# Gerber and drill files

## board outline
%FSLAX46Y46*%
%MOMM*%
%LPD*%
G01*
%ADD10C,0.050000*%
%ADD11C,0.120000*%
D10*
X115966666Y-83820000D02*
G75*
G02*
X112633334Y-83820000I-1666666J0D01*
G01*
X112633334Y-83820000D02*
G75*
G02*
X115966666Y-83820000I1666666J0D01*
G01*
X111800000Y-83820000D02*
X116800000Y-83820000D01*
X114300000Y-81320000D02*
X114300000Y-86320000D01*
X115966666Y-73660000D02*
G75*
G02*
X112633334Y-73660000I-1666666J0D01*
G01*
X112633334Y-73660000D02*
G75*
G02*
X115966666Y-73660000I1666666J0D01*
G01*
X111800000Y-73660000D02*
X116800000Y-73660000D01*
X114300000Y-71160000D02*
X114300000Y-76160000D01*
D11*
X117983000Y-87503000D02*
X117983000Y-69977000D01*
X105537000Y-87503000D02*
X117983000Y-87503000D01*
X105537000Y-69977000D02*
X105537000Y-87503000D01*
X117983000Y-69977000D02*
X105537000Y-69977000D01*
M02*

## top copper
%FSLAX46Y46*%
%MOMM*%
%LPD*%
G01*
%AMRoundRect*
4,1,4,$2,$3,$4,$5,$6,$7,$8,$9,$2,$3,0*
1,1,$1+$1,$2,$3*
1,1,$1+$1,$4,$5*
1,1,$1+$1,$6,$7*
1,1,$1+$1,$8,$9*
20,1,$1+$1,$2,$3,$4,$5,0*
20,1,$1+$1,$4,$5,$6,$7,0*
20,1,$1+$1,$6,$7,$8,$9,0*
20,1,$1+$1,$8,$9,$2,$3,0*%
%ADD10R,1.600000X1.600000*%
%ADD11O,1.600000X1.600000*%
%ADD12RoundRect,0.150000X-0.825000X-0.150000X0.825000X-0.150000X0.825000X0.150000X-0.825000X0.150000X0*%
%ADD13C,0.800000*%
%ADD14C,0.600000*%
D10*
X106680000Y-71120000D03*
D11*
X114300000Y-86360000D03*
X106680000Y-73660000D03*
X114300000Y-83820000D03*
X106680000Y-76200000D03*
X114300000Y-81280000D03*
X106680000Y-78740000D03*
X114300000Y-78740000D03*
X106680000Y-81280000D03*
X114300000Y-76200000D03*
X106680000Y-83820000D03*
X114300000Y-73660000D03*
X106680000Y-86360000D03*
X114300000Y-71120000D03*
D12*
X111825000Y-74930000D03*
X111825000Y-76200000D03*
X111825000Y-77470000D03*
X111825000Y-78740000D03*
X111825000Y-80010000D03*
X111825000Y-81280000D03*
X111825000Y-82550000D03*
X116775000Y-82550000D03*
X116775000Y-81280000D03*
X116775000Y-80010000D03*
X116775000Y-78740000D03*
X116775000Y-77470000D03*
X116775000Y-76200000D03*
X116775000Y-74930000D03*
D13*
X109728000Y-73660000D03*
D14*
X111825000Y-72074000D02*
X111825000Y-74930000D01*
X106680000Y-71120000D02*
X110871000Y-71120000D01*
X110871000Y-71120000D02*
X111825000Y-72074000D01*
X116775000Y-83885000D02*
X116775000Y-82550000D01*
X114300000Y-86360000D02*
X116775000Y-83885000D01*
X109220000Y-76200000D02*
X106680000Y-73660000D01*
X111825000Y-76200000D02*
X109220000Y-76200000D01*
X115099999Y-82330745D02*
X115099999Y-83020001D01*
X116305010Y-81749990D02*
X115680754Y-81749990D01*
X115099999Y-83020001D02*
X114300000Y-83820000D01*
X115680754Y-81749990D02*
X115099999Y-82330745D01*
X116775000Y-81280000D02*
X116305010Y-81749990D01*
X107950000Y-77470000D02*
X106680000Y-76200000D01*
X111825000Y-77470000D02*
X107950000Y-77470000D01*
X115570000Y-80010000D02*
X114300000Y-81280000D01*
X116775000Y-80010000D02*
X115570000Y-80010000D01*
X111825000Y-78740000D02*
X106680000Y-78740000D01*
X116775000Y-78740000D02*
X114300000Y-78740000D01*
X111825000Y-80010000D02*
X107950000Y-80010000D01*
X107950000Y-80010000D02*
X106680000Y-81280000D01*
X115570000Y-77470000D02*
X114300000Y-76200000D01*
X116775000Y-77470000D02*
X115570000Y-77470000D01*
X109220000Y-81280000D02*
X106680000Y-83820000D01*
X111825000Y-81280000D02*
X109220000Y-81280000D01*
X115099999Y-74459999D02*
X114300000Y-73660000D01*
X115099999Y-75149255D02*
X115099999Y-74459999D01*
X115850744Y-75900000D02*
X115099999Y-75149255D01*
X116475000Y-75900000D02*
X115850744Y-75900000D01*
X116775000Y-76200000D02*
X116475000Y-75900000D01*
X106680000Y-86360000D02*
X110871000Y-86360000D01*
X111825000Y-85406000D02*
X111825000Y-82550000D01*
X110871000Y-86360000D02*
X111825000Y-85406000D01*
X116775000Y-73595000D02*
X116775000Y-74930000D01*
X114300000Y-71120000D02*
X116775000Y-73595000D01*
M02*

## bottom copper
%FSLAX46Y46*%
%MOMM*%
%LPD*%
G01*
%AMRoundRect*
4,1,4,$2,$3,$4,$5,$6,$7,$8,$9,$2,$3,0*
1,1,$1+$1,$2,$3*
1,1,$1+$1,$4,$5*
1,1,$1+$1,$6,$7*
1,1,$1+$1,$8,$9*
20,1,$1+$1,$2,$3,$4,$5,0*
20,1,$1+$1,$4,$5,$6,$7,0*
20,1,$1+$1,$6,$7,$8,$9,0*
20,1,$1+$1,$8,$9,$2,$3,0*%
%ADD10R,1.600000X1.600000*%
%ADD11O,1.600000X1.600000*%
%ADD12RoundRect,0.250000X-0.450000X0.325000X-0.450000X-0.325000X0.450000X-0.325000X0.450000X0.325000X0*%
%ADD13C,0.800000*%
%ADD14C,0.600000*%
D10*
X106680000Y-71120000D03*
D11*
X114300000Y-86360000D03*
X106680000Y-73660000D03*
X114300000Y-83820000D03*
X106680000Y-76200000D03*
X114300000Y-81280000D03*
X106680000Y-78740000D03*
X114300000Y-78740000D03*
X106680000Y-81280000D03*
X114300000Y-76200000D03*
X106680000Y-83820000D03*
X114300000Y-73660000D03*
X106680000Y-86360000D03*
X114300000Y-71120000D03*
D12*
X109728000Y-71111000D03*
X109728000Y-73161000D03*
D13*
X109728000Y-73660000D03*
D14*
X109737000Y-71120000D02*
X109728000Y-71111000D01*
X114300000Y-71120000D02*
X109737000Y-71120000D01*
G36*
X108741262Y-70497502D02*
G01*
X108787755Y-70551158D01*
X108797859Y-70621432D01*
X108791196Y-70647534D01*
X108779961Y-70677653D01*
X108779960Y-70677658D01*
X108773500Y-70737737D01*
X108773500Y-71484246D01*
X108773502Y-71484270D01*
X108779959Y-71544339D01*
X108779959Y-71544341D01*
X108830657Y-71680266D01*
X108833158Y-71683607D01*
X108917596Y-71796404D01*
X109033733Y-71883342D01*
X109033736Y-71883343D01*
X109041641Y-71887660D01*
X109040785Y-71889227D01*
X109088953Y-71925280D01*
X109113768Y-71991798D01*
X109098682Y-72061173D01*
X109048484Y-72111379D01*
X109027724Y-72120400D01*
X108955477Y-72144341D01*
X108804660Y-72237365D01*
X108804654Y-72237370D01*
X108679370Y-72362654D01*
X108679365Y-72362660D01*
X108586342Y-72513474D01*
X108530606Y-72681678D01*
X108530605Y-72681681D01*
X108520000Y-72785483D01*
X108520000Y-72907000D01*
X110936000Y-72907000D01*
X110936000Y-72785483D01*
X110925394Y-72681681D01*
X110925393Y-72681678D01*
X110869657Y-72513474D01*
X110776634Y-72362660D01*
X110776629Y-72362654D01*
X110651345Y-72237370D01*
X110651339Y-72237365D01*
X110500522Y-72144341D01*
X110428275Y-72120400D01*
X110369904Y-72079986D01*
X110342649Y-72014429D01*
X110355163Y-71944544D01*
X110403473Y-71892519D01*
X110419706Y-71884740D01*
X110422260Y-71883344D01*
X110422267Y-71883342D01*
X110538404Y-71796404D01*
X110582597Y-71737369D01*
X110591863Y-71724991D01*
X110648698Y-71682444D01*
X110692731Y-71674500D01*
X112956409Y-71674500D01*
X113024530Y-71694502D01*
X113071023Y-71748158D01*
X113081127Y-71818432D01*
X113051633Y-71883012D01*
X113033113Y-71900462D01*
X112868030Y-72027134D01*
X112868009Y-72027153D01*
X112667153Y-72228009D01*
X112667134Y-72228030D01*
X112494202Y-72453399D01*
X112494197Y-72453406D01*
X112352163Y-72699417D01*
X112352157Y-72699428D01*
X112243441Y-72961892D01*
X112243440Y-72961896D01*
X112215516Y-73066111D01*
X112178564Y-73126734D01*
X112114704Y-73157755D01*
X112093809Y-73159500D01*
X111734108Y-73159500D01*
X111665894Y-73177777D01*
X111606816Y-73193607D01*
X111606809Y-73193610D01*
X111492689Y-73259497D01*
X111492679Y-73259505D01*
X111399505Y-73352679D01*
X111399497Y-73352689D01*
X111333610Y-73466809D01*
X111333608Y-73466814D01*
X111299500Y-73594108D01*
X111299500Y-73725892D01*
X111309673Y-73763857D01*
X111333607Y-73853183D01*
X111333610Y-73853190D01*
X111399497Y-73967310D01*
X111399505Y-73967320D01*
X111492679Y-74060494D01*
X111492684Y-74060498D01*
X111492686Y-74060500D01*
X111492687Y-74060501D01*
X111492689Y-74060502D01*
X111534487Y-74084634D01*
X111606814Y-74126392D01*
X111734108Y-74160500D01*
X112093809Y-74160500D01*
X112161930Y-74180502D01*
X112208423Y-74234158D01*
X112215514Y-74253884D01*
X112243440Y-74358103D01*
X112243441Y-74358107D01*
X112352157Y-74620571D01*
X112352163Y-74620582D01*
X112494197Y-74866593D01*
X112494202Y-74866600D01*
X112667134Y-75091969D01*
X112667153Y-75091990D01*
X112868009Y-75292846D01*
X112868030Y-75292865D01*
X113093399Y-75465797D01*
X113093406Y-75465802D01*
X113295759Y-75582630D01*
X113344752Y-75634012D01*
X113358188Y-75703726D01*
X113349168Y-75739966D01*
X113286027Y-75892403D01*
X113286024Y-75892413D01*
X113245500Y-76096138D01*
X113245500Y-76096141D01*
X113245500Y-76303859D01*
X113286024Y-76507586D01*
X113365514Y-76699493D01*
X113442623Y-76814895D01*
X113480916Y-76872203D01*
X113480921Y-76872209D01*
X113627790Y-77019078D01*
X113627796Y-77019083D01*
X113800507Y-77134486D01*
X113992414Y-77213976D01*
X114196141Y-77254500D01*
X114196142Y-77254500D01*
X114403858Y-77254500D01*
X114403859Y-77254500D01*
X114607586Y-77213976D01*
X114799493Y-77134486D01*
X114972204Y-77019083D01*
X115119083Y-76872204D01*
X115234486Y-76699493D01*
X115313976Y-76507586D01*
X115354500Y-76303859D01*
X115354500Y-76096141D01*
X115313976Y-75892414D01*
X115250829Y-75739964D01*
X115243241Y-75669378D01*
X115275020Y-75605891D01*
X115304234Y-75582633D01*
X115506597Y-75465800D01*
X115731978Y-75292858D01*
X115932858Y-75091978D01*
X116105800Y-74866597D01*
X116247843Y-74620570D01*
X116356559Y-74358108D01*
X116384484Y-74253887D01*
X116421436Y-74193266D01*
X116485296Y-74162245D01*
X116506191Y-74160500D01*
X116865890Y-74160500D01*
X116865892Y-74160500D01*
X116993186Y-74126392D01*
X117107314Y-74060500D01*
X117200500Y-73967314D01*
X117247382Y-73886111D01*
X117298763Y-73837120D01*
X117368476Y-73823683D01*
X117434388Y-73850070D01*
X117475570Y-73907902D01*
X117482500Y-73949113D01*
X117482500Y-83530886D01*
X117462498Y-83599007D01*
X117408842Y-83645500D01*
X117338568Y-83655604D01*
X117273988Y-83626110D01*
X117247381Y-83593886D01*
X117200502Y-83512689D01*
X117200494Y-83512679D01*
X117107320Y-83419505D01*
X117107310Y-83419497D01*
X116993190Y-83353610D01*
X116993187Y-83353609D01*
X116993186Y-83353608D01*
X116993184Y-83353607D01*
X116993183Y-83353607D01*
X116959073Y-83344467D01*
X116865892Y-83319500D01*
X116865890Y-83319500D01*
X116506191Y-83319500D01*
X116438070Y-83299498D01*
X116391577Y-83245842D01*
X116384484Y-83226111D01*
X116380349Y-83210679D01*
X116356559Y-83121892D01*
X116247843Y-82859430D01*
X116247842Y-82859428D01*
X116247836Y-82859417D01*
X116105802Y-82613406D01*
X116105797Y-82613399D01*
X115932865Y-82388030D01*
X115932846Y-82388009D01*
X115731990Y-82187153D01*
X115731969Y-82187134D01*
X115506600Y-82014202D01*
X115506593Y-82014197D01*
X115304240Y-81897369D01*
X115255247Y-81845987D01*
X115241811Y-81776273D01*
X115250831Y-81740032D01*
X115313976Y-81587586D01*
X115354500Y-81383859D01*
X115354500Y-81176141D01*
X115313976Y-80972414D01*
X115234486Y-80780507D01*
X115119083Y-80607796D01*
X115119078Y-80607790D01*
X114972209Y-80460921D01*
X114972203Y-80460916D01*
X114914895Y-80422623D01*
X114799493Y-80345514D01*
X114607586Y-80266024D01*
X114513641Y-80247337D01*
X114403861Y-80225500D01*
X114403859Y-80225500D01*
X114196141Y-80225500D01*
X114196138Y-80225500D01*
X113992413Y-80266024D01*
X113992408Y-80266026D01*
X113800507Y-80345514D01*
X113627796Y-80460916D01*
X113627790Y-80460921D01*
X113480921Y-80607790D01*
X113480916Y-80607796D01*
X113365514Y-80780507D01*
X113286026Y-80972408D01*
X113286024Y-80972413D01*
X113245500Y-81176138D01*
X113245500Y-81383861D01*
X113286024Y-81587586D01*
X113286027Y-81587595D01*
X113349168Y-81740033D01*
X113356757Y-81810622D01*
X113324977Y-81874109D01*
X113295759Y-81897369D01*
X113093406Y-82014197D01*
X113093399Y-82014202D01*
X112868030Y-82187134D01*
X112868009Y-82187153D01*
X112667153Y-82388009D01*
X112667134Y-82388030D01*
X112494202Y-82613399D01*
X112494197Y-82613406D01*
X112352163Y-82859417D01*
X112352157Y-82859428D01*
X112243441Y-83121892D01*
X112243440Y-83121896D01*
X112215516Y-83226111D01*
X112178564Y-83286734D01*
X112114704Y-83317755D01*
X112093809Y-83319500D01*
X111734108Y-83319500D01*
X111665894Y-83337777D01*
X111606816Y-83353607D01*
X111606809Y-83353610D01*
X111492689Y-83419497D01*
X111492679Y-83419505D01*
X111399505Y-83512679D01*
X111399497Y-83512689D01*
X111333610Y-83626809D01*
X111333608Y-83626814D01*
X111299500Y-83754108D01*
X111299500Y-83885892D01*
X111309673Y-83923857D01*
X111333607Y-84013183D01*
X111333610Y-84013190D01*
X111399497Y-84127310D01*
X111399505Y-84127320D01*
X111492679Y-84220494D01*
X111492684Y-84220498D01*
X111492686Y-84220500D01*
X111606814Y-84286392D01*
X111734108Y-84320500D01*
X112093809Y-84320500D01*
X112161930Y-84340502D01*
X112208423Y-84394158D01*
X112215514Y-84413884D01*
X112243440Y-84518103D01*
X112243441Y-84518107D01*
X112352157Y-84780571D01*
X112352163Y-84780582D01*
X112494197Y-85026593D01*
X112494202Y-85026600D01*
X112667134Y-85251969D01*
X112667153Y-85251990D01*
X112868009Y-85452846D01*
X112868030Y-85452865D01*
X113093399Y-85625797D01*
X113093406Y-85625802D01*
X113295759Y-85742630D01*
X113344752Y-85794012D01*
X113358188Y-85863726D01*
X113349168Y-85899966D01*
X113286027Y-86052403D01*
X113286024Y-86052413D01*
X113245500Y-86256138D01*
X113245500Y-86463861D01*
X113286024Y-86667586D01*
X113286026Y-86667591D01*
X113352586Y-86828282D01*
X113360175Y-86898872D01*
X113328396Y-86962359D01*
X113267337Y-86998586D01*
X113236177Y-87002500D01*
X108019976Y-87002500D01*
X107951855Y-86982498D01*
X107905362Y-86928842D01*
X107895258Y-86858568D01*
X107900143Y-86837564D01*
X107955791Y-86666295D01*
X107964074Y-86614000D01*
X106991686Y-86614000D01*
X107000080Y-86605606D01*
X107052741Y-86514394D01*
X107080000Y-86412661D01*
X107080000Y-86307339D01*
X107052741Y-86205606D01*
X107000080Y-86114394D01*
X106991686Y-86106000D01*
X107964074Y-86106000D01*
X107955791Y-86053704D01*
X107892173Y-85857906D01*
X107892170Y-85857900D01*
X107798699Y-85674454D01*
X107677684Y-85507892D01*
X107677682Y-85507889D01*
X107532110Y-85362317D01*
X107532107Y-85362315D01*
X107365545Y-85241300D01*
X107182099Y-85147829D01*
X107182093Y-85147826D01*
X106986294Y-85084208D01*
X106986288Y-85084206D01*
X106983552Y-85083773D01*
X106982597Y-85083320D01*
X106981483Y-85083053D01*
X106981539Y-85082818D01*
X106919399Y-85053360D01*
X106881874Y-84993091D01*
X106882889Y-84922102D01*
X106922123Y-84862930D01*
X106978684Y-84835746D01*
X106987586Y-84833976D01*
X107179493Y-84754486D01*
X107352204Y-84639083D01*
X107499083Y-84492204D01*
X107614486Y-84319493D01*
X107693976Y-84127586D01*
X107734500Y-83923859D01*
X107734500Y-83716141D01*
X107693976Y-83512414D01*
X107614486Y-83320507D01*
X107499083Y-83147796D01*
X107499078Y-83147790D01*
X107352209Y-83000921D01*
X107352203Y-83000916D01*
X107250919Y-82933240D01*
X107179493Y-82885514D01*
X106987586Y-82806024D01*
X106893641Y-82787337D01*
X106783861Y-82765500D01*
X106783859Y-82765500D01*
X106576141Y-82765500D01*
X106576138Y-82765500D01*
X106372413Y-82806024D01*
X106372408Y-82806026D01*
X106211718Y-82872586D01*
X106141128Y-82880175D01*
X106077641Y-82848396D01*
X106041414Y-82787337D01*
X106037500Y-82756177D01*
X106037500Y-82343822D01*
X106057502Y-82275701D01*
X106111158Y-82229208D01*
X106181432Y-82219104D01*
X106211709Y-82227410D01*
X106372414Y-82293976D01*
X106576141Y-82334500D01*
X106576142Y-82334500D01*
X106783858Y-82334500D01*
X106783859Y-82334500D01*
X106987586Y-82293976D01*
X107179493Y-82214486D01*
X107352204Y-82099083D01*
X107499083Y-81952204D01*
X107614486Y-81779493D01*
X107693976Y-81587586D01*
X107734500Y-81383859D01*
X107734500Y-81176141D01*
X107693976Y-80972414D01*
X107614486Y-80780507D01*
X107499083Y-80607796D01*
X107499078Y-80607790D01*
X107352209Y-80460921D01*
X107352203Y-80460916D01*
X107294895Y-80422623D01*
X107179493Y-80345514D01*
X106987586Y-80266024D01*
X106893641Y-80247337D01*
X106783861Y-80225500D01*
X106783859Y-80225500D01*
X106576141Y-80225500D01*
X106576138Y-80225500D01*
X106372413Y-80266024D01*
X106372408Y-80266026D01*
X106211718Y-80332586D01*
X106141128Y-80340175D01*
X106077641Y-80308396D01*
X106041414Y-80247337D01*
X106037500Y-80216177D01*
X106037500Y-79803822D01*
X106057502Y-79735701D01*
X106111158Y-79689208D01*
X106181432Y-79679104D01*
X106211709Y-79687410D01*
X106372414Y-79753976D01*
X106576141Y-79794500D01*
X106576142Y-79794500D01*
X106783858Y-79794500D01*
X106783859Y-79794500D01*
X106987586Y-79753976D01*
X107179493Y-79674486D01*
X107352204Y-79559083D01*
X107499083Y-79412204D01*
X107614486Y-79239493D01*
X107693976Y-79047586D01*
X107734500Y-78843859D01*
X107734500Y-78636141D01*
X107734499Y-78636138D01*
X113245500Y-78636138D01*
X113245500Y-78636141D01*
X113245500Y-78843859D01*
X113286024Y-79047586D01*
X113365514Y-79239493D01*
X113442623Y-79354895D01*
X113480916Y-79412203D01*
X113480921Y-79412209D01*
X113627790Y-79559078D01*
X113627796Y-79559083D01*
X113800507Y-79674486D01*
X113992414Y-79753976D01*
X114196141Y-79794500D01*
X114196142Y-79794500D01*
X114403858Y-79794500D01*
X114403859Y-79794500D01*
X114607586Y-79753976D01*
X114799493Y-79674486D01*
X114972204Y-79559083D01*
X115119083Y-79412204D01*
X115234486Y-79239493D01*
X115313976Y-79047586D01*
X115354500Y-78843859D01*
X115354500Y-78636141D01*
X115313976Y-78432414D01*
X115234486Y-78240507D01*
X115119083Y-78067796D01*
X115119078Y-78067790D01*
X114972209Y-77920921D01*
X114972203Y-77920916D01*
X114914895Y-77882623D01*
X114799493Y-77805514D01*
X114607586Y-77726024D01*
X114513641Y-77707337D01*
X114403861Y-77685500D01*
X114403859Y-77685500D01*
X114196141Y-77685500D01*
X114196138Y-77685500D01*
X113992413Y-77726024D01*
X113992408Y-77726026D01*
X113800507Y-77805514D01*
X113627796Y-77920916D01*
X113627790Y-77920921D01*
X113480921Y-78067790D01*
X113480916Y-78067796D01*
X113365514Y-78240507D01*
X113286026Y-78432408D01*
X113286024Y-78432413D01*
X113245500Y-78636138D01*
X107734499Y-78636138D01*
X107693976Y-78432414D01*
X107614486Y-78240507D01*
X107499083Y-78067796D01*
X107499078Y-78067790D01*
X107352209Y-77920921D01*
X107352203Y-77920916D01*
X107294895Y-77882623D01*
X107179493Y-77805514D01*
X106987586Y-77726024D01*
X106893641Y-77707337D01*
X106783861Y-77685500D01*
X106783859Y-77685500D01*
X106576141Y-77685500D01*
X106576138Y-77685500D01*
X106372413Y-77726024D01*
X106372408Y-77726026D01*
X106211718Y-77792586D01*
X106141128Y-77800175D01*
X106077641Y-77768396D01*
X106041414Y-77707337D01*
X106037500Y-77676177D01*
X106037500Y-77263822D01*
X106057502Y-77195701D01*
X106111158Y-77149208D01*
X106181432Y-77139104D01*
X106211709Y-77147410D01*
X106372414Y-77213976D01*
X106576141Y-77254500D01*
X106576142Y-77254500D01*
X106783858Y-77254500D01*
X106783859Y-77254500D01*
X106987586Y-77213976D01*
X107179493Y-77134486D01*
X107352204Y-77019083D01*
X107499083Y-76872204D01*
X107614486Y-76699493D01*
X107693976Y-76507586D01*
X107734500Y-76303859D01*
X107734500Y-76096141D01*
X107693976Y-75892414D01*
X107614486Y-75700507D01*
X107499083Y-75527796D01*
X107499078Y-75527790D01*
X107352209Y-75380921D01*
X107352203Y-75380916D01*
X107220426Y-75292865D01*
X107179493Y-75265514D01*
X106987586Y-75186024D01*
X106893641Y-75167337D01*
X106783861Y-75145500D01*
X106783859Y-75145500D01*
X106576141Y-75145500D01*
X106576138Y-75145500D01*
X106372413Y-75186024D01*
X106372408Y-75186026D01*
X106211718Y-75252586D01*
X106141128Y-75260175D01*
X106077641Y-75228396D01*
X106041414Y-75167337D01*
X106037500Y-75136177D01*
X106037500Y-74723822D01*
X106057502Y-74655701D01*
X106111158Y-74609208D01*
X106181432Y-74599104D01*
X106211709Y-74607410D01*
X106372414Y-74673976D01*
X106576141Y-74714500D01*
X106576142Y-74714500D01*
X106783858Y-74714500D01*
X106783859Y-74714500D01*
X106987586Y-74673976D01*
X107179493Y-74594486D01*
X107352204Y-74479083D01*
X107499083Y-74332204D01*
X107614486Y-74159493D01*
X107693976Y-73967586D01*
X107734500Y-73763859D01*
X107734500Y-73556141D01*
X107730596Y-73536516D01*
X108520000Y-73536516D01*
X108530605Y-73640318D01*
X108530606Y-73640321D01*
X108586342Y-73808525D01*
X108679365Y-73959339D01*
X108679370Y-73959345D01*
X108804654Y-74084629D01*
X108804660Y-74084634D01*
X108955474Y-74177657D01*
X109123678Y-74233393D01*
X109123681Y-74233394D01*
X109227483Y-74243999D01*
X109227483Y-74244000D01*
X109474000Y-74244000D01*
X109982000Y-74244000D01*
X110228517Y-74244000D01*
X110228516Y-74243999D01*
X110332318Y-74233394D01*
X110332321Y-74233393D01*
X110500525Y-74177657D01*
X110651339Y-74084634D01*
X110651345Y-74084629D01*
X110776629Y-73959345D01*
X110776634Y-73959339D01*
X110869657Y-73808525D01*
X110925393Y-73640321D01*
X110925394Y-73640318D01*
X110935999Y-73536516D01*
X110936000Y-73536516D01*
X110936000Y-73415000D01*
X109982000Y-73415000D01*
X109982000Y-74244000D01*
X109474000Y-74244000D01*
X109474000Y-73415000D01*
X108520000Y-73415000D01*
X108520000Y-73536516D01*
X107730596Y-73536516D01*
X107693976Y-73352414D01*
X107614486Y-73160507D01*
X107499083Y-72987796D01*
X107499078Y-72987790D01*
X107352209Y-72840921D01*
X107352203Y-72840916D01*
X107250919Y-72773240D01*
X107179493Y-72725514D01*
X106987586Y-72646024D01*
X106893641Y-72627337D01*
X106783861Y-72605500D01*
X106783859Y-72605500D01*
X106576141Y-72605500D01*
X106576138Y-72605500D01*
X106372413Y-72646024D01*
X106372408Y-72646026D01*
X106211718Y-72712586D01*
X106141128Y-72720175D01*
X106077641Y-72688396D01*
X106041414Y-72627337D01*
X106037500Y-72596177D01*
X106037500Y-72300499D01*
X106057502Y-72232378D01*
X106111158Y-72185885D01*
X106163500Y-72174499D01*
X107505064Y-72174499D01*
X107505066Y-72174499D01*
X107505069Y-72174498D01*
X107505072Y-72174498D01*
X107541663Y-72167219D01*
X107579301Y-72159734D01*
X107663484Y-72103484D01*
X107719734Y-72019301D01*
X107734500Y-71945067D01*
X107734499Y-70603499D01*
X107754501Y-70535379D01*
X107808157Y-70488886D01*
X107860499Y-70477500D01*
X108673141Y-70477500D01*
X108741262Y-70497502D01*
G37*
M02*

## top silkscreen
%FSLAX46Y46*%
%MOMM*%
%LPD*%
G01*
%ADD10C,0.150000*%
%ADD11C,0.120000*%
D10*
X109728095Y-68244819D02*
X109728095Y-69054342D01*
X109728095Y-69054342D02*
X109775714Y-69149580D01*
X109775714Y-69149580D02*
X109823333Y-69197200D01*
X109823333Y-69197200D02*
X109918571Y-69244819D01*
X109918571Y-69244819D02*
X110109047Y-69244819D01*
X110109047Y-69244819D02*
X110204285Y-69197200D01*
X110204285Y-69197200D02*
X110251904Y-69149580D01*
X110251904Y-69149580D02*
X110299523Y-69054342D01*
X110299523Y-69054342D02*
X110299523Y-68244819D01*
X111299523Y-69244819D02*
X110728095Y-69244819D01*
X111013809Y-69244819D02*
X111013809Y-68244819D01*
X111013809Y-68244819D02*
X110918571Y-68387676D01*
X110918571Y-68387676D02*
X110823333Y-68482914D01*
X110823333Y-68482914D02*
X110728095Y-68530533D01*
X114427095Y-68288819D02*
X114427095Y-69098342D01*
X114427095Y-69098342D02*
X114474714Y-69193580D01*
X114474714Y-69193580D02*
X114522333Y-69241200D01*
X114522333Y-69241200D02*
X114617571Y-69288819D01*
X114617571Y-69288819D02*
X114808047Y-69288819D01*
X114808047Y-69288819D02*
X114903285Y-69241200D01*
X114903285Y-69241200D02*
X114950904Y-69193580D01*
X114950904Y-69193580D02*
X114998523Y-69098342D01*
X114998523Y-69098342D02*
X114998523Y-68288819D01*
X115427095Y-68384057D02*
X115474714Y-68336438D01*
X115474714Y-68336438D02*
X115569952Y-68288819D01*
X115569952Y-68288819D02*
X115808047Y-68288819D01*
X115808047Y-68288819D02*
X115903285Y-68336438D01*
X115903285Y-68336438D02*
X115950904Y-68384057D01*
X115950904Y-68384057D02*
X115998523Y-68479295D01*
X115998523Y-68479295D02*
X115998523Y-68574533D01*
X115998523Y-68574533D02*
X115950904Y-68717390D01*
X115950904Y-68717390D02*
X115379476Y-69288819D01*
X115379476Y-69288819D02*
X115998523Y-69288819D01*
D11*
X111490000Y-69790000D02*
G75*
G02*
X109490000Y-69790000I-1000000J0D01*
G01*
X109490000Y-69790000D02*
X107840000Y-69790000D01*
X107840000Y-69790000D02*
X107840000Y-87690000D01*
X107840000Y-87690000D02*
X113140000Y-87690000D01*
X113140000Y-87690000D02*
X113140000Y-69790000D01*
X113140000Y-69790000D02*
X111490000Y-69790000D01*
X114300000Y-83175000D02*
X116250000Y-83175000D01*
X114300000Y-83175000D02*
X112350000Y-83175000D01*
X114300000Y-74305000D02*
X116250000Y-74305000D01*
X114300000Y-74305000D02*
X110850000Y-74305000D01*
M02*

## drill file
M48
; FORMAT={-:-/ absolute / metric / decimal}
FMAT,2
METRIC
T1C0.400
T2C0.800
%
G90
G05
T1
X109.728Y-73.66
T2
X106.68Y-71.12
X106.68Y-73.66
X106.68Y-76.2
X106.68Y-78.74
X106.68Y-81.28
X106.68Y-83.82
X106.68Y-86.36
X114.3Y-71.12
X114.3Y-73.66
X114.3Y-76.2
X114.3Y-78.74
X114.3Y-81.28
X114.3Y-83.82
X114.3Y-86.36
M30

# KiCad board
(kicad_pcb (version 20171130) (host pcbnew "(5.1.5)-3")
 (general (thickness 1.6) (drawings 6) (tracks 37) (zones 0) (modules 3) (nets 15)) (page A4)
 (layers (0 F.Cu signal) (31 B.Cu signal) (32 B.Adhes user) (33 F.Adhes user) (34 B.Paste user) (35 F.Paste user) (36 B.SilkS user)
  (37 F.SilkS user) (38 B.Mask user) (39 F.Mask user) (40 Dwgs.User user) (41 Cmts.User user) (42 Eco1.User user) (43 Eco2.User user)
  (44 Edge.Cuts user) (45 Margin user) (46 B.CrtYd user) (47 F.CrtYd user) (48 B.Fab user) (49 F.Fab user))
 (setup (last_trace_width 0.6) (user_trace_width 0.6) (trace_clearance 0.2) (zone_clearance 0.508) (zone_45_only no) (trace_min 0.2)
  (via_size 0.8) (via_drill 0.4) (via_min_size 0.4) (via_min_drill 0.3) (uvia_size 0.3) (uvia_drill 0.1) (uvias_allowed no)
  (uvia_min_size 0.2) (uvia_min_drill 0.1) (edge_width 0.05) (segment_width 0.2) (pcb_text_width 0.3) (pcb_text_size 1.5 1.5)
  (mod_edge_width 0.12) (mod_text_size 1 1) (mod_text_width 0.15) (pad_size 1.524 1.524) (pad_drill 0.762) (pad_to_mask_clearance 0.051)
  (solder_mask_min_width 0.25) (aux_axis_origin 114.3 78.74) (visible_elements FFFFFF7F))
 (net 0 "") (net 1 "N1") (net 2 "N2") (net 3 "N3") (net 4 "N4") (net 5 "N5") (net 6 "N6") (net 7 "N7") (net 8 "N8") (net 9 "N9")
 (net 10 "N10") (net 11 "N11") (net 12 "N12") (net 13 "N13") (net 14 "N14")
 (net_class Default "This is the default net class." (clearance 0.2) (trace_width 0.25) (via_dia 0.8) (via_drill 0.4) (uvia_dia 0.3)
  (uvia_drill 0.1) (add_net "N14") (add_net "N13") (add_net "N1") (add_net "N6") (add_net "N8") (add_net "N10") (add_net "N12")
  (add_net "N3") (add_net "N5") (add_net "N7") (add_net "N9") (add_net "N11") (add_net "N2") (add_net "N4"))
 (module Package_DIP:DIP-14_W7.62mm (layer F.Cu) (at 106.68 71.12)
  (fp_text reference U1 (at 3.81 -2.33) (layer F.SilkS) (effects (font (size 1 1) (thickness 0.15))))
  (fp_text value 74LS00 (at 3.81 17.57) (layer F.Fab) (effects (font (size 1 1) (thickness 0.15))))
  (fp_arc (start 3.81 -1.33) (end 2.81 -1.33) (angle -180) (layer F.SilkS) (width 0.12))
  (fp_line (start 2.81 -1.33) (end 1.16 -1.33) (layer F.SilkS) (width 0.12))
  (fp_line (start 1.16 -1.33) (end 1.16 16.57) (layer F.SilkS) (width 0.12))
  (fp_line (start 1.16 16.57) (end 6.46 16.57) (layer F.SilkS) (width 0.12))
  (fp_line (start 6.46 16.57) (end 6.46 -1.33) (layer F.SilkS) (width 0.12))
  (fp_line (start 6.46 -1.33) (end 4.81 -1.33) (layer F.SilkS) (width 0.12))
  (pad 1 thru_hole rect (at 0 0) (size 1.6 1.6) (drill 0.8) (layers *.Cu *.Mask) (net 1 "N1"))
  (pad 8 thru_hole oval (at 7.62 15.24) (size 1.6 1.6) (drill 0.8) (layers *.Cu *.Mask) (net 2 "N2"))
  (pad 2 thru_hole oval (at 0 2.54) (size 1.6 1.6) (drill 0.8) (layers *.Cu *.Mask) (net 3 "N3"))
  (pad 9 thru_hole oval (at 7.62 12.7) (size 1.6 1.6) (drill 0.8) (layers *.Cu *.Mask) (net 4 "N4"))
  (pad 3 thru_hole oval (at 0 5.08) (size 1.6 1.6) (drill 0.8) (layers *.Cu *.Mask) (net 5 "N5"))
  (pad 10 thru_hole oval (at 7.62 10.16) (size 1.6 1.6) (drill 0.8) (layers *.Cu *.Mask) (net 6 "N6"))
  (pad 4 thru_hole oval (at 0 7.62) (size 1.6 1.6) (drill 0.8) (layers *.Cu *.Mask) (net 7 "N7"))
  (pad 11 thru_hole oval (at 7.62 7.62) (size 1.6 1.6) (drill 0.8) (layers *.Cu *.Mask) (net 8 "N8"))
  (pad 5 thru_hole oval (at 0 10.16) (size 1.6 1.6) (drill 0.8) (layers *.Cu *.Mask) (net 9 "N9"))
  (pad 12 thru_hole oval (at 7.62 5.08) (size 1.6 1.6) (drill 0.8) (layers *.Cu *.Mask) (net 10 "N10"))
  (pad 6 thru_hole oval (at 0 12.7) (size 1.6 1.6) (drill 0.8) (layers *.Cu *.Mask) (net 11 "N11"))
  (pad 13 thru_hole oval (at 7.62 2.54) (size 1.6 1.6) (drill 0.8) (layers *.Cu *.Mask) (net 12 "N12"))
  (pad 7 thru_hole oval (at 0 15.24) (size 1.6 1.6) (drill 0.8) (layers *.Cu *.Mask) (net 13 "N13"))
  (pad 14 thru_hole oval (at 7.62 0) (size 1.6 1.6) (drill 0.8) (layers *.Cu *.Mask) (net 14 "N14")))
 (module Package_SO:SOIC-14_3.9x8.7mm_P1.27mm (layer F.Cu) (at 114.3 78.74)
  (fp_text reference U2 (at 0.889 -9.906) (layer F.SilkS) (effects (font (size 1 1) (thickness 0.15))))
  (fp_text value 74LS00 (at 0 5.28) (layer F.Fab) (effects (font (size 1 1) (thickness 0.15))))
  (fp_line (start 0 4.435) (end 1.95 4.435) (layer F.SilkS) (width 0.12))
  (fp_line (start 0 4.435) (end -1.95 4.435) (layer F.SilkS) (width 0.12))
  (fp_line (start 0 -4.435) (end 1.95 -4.435) (layer F.SilkS) (width 0.12))
  (fp_line (start 0 -4.435) (end -3.45 -4.435) (layer F.SilkS) (width 0.12))
  (pad 1 smd roundrect (at -2.475 -3.81) (size 1.95 0.6) (layers F.Cu F.Paste F.Mask) (roundrect_rratio 0.25) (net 1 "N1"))
  (pad 2 smd roundrect (at -2.475 -2.54) (size 1.95 0.6) (layers F.Cu F.Paste F.Mask) (roundrect_rratio 0.25) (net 3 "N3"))
  (pad 3 smd roundrect (at -2.475 -1.27) (size 1.95 0.6) (layers F.Cu F.Paste F.Mask) (roundrect_rratio 0.25) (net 5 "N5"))
  (pad 4 smd roundrect (at -2.475 0) (size 1.95 0.6) (layers F.Cu F.Paste F.Mask) (roundrect_rratio 0.25) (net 7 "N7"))
  (pad 5 smd roundrect (at -2.475 1.27) (size 1.95 0.6) (layers F.Cu F.Paste F.Mask) (roundrect_rratio 0.25) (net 9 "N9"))
  (pad 6 smd roundrect (at -2.475 2.54) (size 1.95 0.6) (layers F.Cu F.Paste F.Mask) (roundrect_rratio 0.25) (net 11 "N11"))
  (pad 7 smd roundrect (at -2.475 3.81) (size 1.95 0.6) (layers F.Cu F.Paste F.Mask) (roundrect_rratio 0.25) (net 13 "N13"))
  (pad 8 smd roundrect (at 2.475 3.81) (size 1.95 0.6) (layers F.Cu F.Paste F.Mask) (roundrect_rratio 0.25) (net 2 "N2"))
  (pad 9 smd roundrect (at 2.475 2.54) (size 1.95 0.6) (layers F.Cu F.Paste F.Mask) (roundrect_rratio 0.25) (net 4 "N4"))
  (pad 10 smd roundrect (at 2.475 1.27) (size 1.95 0.6) (layers F.Cu F.Paste F.Mask) (roundrect_rratio 0.25) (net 6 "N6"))
  (pad 11 smd roundrect (at 2.475 0) (size 1.95 0.6) (layers F.Cu F.Paste F.Mask) (roundrect_rratio 0.25) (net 8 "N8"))
  (pad 12 smd roundrect (at 2.475 -1.27) (size 1.95 0.6) (layers F.Cu F.Paste F.Mask) (roundrect_rratio 0.25) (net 10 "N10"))
  (pad 13 smd roundrect (at 2.475 -2.54) (size 1.95 0.6) (layers F.Cu F.Paste F.Mask) (roundrect_rratio 0.25) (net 12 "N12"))
  (pad 14 smd roundrect (at 2.475 -3.81) (size 1.95 0.6) (layers F.Cu F.Paste F.Mask) (roundrect_rratio 0.25) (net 14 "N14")))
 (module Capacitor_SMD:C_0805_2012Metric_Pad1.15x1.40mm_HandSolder (layer B.Cu) (at 109.728 72.136 270)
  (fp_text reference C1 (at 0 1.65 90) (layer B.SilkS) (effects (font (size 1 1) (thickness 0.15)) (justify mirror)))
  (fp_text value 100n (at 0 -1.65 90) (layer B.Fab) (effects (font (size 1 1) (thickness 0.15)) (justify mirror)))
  (pad 1 smd roundrect (at -1.025 0 270) (size 1.15 1.4) (layers B.Cu B.Paste B.Mask) (roundrect_rratio 0.217391) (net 14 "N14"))
  (pad 2 smd roundrect (at 1.025 0 270) (size 1.15 1.4) (layers B.Cu B.Paste B.Mask) (roundrect_rratio 0.217391) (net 13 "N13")))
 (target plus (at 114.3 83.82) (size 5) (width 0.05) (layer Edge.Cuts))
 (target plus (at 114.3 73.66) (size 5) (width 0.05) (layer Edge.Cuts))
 (gr_line (start 117.983 87.503) (end 117.983 69.977) (layer Edge.Cuts) (width 0.12))
 (gr_line (start 105.537 87.503) (end 117.983 87.503) (layer Edge.Cuts) (width 0.12))
 (gr_line (start 105.537 69.977) (end 105.537 87.503) (layer Edge.Cuts) (width 0.12))
 (gr_line (start 117.983 69.977) (end 105.537 69.977) (layer Edge.Cuts) (width 0.12))
 (via (at 109.728 73.66) (size 0.8) (drill 0.4) (layers F.Cu B.Cu) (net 13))
 (segment (start 111.825 72.074) (end 111.825 74.93) (width 0.6) (layer F.Cu) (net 1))
 (segment (start 106.68 71.12) (end 110.871 71.12) (width 0.6) (layer F.Cu) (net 1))
 (segment (start 110.871 71.12) (end 111.825 72.074) (width 0.6) (layer F.Cu) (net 1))
 (segment (start 116.775 83.885) (end 116.775 82.55) (width 0.6) (layer F.Cu) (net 2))
 (segment (start 114.3 86.36) (end 116.775 83.885) (width 0.6) (layer F.Cu) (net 2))
 (segment (start 109.22 76.2) (end 106.68 73.66) (width 0.6) (layer F.Cu) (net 3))
 (segment (start 111.825 76.2) (end 109.22 76.2) (width 0.6) (layer F.Cu) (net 3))
 (segment (start 115.099999 82.330745) (end 115.099999 83.020001) (width 0.6) (layer F.Cu) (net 4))
 (segment (start 116.30501 81.74999) (end 115.680754 81.74999) (width 0.6) (layer F.Cu) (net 4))
 (segment (start 115.099999 83.020001) (end 114.3 83.82) (width 0.6) (layer F.Cu) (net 4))
 (segment (start 115.680754 81.74999) (end 115.099999 82.330745) (width 0.6) (layer F.Cu) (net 4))
 (segment (start 116.775 81.28) (end 116.30501 81.74999) (width 0.6) (layer F.Cu) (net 4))
 (segment (start 107.95 77.47) (end 106.68 76.2) (width 0.6) (layer F.Cu) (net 5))
 (segment (start 111.825 77.47) (end 107.95 77.47) (width 0.6) (layer F.Cu) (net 5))
 (segment (start 115.57 80.01) (end 114.3 81.28) (width 0.6) (layer F.Cu) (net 6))
 (segment (start 116.775 80.01) (end 115.57 80.01) (width 0.6) (layer F.Cu) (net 6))
 (segment (start 111.825 78.74) (end 106.68 78.74) (width 0.6) (layer F.Cu) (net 7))
 (segment (start 116.775 78.74) (end 114.3 78.74) (width 0.6) (layer F.Cu) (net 8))
 (segment (start 111.825 80.01) (end 107.95 80.01) (width 0.6) (layer F.Cu) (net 9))
 (segment (start 107.95 80.01) (end 106.68 81.28) (width 0.6) (layer F.Cu) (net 9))
 (segment (start 115.57 77.47) (end 114.3 76.2) (width 0.6) (layer F.Cu) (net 10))
 (segment (start 116.775 77.47) (end 115.57 77.47) (width 0.6) (layer F.Cu) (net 10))
 (segment (start 109.22 81.28) (end 106.68 83.82) (width 0.6) (layer F.Cu) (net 11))
 (segment (start 111.825 81.28) (end 109.22 81.28) (width 0.6) (layer F.Cu) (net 11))
 (segment (start 115.099999 74.459999) (end 114.3 73.66) (width 0.6) (layer F.Cu) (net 12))
 (segment (start 115.099999 75.149255) (end 115.099999 74.459999) (width 0.6) (layer F.Cu) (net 12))
 (segment (start 115.850744 75.9) (end 115.099999 75.149255) (width 0.6) (layer F.Cu) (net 12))
 (segment (start 116.475 75.9) (end 115.850744 75.9) (width 0.6) (layer F.Cu) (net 12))
 (segment (start 116.775 76.2) (end 116.475 75.9) (width 0.6) (layer F.Cu) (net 12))
 (segment (start 106.68 86.36) (end 110.871 86.36) (width 0.6) (layer F.Cu) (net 13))
 (segment (start 111.825 85.406) (end 111.825 82.55) (width 0.6) (layer F.Cu) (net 13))
 (segment (start 110.871 86.36) (end 111.825 85.406) (width 0.6) (layer F.Cu) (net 13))
 (segment (start 116.775 73.595) (end 116.775 74.93) (width 0.6) (layer F.Cu) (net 14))
 (segment (start 114.3 71.12) (end 116.775 73.595) (width 0.6) (layer F.Cu) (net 14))
 (segment (start 109.737 71.12) (end 109.728 71.111) (width 0.6) (layer B.Cu) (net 14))
 (segment (start 114.3 71.12) (end 109.737 71.12) (width 0.6) (layer B.Cu) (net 14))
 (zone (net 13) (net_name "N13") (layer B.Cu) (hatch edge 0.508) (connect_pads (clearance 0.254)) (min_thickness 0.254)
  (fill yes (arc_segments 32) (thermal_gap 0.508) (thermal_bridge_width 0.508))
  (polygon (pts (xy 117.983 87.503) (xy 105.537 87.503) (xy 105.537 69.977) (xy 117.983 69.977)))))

